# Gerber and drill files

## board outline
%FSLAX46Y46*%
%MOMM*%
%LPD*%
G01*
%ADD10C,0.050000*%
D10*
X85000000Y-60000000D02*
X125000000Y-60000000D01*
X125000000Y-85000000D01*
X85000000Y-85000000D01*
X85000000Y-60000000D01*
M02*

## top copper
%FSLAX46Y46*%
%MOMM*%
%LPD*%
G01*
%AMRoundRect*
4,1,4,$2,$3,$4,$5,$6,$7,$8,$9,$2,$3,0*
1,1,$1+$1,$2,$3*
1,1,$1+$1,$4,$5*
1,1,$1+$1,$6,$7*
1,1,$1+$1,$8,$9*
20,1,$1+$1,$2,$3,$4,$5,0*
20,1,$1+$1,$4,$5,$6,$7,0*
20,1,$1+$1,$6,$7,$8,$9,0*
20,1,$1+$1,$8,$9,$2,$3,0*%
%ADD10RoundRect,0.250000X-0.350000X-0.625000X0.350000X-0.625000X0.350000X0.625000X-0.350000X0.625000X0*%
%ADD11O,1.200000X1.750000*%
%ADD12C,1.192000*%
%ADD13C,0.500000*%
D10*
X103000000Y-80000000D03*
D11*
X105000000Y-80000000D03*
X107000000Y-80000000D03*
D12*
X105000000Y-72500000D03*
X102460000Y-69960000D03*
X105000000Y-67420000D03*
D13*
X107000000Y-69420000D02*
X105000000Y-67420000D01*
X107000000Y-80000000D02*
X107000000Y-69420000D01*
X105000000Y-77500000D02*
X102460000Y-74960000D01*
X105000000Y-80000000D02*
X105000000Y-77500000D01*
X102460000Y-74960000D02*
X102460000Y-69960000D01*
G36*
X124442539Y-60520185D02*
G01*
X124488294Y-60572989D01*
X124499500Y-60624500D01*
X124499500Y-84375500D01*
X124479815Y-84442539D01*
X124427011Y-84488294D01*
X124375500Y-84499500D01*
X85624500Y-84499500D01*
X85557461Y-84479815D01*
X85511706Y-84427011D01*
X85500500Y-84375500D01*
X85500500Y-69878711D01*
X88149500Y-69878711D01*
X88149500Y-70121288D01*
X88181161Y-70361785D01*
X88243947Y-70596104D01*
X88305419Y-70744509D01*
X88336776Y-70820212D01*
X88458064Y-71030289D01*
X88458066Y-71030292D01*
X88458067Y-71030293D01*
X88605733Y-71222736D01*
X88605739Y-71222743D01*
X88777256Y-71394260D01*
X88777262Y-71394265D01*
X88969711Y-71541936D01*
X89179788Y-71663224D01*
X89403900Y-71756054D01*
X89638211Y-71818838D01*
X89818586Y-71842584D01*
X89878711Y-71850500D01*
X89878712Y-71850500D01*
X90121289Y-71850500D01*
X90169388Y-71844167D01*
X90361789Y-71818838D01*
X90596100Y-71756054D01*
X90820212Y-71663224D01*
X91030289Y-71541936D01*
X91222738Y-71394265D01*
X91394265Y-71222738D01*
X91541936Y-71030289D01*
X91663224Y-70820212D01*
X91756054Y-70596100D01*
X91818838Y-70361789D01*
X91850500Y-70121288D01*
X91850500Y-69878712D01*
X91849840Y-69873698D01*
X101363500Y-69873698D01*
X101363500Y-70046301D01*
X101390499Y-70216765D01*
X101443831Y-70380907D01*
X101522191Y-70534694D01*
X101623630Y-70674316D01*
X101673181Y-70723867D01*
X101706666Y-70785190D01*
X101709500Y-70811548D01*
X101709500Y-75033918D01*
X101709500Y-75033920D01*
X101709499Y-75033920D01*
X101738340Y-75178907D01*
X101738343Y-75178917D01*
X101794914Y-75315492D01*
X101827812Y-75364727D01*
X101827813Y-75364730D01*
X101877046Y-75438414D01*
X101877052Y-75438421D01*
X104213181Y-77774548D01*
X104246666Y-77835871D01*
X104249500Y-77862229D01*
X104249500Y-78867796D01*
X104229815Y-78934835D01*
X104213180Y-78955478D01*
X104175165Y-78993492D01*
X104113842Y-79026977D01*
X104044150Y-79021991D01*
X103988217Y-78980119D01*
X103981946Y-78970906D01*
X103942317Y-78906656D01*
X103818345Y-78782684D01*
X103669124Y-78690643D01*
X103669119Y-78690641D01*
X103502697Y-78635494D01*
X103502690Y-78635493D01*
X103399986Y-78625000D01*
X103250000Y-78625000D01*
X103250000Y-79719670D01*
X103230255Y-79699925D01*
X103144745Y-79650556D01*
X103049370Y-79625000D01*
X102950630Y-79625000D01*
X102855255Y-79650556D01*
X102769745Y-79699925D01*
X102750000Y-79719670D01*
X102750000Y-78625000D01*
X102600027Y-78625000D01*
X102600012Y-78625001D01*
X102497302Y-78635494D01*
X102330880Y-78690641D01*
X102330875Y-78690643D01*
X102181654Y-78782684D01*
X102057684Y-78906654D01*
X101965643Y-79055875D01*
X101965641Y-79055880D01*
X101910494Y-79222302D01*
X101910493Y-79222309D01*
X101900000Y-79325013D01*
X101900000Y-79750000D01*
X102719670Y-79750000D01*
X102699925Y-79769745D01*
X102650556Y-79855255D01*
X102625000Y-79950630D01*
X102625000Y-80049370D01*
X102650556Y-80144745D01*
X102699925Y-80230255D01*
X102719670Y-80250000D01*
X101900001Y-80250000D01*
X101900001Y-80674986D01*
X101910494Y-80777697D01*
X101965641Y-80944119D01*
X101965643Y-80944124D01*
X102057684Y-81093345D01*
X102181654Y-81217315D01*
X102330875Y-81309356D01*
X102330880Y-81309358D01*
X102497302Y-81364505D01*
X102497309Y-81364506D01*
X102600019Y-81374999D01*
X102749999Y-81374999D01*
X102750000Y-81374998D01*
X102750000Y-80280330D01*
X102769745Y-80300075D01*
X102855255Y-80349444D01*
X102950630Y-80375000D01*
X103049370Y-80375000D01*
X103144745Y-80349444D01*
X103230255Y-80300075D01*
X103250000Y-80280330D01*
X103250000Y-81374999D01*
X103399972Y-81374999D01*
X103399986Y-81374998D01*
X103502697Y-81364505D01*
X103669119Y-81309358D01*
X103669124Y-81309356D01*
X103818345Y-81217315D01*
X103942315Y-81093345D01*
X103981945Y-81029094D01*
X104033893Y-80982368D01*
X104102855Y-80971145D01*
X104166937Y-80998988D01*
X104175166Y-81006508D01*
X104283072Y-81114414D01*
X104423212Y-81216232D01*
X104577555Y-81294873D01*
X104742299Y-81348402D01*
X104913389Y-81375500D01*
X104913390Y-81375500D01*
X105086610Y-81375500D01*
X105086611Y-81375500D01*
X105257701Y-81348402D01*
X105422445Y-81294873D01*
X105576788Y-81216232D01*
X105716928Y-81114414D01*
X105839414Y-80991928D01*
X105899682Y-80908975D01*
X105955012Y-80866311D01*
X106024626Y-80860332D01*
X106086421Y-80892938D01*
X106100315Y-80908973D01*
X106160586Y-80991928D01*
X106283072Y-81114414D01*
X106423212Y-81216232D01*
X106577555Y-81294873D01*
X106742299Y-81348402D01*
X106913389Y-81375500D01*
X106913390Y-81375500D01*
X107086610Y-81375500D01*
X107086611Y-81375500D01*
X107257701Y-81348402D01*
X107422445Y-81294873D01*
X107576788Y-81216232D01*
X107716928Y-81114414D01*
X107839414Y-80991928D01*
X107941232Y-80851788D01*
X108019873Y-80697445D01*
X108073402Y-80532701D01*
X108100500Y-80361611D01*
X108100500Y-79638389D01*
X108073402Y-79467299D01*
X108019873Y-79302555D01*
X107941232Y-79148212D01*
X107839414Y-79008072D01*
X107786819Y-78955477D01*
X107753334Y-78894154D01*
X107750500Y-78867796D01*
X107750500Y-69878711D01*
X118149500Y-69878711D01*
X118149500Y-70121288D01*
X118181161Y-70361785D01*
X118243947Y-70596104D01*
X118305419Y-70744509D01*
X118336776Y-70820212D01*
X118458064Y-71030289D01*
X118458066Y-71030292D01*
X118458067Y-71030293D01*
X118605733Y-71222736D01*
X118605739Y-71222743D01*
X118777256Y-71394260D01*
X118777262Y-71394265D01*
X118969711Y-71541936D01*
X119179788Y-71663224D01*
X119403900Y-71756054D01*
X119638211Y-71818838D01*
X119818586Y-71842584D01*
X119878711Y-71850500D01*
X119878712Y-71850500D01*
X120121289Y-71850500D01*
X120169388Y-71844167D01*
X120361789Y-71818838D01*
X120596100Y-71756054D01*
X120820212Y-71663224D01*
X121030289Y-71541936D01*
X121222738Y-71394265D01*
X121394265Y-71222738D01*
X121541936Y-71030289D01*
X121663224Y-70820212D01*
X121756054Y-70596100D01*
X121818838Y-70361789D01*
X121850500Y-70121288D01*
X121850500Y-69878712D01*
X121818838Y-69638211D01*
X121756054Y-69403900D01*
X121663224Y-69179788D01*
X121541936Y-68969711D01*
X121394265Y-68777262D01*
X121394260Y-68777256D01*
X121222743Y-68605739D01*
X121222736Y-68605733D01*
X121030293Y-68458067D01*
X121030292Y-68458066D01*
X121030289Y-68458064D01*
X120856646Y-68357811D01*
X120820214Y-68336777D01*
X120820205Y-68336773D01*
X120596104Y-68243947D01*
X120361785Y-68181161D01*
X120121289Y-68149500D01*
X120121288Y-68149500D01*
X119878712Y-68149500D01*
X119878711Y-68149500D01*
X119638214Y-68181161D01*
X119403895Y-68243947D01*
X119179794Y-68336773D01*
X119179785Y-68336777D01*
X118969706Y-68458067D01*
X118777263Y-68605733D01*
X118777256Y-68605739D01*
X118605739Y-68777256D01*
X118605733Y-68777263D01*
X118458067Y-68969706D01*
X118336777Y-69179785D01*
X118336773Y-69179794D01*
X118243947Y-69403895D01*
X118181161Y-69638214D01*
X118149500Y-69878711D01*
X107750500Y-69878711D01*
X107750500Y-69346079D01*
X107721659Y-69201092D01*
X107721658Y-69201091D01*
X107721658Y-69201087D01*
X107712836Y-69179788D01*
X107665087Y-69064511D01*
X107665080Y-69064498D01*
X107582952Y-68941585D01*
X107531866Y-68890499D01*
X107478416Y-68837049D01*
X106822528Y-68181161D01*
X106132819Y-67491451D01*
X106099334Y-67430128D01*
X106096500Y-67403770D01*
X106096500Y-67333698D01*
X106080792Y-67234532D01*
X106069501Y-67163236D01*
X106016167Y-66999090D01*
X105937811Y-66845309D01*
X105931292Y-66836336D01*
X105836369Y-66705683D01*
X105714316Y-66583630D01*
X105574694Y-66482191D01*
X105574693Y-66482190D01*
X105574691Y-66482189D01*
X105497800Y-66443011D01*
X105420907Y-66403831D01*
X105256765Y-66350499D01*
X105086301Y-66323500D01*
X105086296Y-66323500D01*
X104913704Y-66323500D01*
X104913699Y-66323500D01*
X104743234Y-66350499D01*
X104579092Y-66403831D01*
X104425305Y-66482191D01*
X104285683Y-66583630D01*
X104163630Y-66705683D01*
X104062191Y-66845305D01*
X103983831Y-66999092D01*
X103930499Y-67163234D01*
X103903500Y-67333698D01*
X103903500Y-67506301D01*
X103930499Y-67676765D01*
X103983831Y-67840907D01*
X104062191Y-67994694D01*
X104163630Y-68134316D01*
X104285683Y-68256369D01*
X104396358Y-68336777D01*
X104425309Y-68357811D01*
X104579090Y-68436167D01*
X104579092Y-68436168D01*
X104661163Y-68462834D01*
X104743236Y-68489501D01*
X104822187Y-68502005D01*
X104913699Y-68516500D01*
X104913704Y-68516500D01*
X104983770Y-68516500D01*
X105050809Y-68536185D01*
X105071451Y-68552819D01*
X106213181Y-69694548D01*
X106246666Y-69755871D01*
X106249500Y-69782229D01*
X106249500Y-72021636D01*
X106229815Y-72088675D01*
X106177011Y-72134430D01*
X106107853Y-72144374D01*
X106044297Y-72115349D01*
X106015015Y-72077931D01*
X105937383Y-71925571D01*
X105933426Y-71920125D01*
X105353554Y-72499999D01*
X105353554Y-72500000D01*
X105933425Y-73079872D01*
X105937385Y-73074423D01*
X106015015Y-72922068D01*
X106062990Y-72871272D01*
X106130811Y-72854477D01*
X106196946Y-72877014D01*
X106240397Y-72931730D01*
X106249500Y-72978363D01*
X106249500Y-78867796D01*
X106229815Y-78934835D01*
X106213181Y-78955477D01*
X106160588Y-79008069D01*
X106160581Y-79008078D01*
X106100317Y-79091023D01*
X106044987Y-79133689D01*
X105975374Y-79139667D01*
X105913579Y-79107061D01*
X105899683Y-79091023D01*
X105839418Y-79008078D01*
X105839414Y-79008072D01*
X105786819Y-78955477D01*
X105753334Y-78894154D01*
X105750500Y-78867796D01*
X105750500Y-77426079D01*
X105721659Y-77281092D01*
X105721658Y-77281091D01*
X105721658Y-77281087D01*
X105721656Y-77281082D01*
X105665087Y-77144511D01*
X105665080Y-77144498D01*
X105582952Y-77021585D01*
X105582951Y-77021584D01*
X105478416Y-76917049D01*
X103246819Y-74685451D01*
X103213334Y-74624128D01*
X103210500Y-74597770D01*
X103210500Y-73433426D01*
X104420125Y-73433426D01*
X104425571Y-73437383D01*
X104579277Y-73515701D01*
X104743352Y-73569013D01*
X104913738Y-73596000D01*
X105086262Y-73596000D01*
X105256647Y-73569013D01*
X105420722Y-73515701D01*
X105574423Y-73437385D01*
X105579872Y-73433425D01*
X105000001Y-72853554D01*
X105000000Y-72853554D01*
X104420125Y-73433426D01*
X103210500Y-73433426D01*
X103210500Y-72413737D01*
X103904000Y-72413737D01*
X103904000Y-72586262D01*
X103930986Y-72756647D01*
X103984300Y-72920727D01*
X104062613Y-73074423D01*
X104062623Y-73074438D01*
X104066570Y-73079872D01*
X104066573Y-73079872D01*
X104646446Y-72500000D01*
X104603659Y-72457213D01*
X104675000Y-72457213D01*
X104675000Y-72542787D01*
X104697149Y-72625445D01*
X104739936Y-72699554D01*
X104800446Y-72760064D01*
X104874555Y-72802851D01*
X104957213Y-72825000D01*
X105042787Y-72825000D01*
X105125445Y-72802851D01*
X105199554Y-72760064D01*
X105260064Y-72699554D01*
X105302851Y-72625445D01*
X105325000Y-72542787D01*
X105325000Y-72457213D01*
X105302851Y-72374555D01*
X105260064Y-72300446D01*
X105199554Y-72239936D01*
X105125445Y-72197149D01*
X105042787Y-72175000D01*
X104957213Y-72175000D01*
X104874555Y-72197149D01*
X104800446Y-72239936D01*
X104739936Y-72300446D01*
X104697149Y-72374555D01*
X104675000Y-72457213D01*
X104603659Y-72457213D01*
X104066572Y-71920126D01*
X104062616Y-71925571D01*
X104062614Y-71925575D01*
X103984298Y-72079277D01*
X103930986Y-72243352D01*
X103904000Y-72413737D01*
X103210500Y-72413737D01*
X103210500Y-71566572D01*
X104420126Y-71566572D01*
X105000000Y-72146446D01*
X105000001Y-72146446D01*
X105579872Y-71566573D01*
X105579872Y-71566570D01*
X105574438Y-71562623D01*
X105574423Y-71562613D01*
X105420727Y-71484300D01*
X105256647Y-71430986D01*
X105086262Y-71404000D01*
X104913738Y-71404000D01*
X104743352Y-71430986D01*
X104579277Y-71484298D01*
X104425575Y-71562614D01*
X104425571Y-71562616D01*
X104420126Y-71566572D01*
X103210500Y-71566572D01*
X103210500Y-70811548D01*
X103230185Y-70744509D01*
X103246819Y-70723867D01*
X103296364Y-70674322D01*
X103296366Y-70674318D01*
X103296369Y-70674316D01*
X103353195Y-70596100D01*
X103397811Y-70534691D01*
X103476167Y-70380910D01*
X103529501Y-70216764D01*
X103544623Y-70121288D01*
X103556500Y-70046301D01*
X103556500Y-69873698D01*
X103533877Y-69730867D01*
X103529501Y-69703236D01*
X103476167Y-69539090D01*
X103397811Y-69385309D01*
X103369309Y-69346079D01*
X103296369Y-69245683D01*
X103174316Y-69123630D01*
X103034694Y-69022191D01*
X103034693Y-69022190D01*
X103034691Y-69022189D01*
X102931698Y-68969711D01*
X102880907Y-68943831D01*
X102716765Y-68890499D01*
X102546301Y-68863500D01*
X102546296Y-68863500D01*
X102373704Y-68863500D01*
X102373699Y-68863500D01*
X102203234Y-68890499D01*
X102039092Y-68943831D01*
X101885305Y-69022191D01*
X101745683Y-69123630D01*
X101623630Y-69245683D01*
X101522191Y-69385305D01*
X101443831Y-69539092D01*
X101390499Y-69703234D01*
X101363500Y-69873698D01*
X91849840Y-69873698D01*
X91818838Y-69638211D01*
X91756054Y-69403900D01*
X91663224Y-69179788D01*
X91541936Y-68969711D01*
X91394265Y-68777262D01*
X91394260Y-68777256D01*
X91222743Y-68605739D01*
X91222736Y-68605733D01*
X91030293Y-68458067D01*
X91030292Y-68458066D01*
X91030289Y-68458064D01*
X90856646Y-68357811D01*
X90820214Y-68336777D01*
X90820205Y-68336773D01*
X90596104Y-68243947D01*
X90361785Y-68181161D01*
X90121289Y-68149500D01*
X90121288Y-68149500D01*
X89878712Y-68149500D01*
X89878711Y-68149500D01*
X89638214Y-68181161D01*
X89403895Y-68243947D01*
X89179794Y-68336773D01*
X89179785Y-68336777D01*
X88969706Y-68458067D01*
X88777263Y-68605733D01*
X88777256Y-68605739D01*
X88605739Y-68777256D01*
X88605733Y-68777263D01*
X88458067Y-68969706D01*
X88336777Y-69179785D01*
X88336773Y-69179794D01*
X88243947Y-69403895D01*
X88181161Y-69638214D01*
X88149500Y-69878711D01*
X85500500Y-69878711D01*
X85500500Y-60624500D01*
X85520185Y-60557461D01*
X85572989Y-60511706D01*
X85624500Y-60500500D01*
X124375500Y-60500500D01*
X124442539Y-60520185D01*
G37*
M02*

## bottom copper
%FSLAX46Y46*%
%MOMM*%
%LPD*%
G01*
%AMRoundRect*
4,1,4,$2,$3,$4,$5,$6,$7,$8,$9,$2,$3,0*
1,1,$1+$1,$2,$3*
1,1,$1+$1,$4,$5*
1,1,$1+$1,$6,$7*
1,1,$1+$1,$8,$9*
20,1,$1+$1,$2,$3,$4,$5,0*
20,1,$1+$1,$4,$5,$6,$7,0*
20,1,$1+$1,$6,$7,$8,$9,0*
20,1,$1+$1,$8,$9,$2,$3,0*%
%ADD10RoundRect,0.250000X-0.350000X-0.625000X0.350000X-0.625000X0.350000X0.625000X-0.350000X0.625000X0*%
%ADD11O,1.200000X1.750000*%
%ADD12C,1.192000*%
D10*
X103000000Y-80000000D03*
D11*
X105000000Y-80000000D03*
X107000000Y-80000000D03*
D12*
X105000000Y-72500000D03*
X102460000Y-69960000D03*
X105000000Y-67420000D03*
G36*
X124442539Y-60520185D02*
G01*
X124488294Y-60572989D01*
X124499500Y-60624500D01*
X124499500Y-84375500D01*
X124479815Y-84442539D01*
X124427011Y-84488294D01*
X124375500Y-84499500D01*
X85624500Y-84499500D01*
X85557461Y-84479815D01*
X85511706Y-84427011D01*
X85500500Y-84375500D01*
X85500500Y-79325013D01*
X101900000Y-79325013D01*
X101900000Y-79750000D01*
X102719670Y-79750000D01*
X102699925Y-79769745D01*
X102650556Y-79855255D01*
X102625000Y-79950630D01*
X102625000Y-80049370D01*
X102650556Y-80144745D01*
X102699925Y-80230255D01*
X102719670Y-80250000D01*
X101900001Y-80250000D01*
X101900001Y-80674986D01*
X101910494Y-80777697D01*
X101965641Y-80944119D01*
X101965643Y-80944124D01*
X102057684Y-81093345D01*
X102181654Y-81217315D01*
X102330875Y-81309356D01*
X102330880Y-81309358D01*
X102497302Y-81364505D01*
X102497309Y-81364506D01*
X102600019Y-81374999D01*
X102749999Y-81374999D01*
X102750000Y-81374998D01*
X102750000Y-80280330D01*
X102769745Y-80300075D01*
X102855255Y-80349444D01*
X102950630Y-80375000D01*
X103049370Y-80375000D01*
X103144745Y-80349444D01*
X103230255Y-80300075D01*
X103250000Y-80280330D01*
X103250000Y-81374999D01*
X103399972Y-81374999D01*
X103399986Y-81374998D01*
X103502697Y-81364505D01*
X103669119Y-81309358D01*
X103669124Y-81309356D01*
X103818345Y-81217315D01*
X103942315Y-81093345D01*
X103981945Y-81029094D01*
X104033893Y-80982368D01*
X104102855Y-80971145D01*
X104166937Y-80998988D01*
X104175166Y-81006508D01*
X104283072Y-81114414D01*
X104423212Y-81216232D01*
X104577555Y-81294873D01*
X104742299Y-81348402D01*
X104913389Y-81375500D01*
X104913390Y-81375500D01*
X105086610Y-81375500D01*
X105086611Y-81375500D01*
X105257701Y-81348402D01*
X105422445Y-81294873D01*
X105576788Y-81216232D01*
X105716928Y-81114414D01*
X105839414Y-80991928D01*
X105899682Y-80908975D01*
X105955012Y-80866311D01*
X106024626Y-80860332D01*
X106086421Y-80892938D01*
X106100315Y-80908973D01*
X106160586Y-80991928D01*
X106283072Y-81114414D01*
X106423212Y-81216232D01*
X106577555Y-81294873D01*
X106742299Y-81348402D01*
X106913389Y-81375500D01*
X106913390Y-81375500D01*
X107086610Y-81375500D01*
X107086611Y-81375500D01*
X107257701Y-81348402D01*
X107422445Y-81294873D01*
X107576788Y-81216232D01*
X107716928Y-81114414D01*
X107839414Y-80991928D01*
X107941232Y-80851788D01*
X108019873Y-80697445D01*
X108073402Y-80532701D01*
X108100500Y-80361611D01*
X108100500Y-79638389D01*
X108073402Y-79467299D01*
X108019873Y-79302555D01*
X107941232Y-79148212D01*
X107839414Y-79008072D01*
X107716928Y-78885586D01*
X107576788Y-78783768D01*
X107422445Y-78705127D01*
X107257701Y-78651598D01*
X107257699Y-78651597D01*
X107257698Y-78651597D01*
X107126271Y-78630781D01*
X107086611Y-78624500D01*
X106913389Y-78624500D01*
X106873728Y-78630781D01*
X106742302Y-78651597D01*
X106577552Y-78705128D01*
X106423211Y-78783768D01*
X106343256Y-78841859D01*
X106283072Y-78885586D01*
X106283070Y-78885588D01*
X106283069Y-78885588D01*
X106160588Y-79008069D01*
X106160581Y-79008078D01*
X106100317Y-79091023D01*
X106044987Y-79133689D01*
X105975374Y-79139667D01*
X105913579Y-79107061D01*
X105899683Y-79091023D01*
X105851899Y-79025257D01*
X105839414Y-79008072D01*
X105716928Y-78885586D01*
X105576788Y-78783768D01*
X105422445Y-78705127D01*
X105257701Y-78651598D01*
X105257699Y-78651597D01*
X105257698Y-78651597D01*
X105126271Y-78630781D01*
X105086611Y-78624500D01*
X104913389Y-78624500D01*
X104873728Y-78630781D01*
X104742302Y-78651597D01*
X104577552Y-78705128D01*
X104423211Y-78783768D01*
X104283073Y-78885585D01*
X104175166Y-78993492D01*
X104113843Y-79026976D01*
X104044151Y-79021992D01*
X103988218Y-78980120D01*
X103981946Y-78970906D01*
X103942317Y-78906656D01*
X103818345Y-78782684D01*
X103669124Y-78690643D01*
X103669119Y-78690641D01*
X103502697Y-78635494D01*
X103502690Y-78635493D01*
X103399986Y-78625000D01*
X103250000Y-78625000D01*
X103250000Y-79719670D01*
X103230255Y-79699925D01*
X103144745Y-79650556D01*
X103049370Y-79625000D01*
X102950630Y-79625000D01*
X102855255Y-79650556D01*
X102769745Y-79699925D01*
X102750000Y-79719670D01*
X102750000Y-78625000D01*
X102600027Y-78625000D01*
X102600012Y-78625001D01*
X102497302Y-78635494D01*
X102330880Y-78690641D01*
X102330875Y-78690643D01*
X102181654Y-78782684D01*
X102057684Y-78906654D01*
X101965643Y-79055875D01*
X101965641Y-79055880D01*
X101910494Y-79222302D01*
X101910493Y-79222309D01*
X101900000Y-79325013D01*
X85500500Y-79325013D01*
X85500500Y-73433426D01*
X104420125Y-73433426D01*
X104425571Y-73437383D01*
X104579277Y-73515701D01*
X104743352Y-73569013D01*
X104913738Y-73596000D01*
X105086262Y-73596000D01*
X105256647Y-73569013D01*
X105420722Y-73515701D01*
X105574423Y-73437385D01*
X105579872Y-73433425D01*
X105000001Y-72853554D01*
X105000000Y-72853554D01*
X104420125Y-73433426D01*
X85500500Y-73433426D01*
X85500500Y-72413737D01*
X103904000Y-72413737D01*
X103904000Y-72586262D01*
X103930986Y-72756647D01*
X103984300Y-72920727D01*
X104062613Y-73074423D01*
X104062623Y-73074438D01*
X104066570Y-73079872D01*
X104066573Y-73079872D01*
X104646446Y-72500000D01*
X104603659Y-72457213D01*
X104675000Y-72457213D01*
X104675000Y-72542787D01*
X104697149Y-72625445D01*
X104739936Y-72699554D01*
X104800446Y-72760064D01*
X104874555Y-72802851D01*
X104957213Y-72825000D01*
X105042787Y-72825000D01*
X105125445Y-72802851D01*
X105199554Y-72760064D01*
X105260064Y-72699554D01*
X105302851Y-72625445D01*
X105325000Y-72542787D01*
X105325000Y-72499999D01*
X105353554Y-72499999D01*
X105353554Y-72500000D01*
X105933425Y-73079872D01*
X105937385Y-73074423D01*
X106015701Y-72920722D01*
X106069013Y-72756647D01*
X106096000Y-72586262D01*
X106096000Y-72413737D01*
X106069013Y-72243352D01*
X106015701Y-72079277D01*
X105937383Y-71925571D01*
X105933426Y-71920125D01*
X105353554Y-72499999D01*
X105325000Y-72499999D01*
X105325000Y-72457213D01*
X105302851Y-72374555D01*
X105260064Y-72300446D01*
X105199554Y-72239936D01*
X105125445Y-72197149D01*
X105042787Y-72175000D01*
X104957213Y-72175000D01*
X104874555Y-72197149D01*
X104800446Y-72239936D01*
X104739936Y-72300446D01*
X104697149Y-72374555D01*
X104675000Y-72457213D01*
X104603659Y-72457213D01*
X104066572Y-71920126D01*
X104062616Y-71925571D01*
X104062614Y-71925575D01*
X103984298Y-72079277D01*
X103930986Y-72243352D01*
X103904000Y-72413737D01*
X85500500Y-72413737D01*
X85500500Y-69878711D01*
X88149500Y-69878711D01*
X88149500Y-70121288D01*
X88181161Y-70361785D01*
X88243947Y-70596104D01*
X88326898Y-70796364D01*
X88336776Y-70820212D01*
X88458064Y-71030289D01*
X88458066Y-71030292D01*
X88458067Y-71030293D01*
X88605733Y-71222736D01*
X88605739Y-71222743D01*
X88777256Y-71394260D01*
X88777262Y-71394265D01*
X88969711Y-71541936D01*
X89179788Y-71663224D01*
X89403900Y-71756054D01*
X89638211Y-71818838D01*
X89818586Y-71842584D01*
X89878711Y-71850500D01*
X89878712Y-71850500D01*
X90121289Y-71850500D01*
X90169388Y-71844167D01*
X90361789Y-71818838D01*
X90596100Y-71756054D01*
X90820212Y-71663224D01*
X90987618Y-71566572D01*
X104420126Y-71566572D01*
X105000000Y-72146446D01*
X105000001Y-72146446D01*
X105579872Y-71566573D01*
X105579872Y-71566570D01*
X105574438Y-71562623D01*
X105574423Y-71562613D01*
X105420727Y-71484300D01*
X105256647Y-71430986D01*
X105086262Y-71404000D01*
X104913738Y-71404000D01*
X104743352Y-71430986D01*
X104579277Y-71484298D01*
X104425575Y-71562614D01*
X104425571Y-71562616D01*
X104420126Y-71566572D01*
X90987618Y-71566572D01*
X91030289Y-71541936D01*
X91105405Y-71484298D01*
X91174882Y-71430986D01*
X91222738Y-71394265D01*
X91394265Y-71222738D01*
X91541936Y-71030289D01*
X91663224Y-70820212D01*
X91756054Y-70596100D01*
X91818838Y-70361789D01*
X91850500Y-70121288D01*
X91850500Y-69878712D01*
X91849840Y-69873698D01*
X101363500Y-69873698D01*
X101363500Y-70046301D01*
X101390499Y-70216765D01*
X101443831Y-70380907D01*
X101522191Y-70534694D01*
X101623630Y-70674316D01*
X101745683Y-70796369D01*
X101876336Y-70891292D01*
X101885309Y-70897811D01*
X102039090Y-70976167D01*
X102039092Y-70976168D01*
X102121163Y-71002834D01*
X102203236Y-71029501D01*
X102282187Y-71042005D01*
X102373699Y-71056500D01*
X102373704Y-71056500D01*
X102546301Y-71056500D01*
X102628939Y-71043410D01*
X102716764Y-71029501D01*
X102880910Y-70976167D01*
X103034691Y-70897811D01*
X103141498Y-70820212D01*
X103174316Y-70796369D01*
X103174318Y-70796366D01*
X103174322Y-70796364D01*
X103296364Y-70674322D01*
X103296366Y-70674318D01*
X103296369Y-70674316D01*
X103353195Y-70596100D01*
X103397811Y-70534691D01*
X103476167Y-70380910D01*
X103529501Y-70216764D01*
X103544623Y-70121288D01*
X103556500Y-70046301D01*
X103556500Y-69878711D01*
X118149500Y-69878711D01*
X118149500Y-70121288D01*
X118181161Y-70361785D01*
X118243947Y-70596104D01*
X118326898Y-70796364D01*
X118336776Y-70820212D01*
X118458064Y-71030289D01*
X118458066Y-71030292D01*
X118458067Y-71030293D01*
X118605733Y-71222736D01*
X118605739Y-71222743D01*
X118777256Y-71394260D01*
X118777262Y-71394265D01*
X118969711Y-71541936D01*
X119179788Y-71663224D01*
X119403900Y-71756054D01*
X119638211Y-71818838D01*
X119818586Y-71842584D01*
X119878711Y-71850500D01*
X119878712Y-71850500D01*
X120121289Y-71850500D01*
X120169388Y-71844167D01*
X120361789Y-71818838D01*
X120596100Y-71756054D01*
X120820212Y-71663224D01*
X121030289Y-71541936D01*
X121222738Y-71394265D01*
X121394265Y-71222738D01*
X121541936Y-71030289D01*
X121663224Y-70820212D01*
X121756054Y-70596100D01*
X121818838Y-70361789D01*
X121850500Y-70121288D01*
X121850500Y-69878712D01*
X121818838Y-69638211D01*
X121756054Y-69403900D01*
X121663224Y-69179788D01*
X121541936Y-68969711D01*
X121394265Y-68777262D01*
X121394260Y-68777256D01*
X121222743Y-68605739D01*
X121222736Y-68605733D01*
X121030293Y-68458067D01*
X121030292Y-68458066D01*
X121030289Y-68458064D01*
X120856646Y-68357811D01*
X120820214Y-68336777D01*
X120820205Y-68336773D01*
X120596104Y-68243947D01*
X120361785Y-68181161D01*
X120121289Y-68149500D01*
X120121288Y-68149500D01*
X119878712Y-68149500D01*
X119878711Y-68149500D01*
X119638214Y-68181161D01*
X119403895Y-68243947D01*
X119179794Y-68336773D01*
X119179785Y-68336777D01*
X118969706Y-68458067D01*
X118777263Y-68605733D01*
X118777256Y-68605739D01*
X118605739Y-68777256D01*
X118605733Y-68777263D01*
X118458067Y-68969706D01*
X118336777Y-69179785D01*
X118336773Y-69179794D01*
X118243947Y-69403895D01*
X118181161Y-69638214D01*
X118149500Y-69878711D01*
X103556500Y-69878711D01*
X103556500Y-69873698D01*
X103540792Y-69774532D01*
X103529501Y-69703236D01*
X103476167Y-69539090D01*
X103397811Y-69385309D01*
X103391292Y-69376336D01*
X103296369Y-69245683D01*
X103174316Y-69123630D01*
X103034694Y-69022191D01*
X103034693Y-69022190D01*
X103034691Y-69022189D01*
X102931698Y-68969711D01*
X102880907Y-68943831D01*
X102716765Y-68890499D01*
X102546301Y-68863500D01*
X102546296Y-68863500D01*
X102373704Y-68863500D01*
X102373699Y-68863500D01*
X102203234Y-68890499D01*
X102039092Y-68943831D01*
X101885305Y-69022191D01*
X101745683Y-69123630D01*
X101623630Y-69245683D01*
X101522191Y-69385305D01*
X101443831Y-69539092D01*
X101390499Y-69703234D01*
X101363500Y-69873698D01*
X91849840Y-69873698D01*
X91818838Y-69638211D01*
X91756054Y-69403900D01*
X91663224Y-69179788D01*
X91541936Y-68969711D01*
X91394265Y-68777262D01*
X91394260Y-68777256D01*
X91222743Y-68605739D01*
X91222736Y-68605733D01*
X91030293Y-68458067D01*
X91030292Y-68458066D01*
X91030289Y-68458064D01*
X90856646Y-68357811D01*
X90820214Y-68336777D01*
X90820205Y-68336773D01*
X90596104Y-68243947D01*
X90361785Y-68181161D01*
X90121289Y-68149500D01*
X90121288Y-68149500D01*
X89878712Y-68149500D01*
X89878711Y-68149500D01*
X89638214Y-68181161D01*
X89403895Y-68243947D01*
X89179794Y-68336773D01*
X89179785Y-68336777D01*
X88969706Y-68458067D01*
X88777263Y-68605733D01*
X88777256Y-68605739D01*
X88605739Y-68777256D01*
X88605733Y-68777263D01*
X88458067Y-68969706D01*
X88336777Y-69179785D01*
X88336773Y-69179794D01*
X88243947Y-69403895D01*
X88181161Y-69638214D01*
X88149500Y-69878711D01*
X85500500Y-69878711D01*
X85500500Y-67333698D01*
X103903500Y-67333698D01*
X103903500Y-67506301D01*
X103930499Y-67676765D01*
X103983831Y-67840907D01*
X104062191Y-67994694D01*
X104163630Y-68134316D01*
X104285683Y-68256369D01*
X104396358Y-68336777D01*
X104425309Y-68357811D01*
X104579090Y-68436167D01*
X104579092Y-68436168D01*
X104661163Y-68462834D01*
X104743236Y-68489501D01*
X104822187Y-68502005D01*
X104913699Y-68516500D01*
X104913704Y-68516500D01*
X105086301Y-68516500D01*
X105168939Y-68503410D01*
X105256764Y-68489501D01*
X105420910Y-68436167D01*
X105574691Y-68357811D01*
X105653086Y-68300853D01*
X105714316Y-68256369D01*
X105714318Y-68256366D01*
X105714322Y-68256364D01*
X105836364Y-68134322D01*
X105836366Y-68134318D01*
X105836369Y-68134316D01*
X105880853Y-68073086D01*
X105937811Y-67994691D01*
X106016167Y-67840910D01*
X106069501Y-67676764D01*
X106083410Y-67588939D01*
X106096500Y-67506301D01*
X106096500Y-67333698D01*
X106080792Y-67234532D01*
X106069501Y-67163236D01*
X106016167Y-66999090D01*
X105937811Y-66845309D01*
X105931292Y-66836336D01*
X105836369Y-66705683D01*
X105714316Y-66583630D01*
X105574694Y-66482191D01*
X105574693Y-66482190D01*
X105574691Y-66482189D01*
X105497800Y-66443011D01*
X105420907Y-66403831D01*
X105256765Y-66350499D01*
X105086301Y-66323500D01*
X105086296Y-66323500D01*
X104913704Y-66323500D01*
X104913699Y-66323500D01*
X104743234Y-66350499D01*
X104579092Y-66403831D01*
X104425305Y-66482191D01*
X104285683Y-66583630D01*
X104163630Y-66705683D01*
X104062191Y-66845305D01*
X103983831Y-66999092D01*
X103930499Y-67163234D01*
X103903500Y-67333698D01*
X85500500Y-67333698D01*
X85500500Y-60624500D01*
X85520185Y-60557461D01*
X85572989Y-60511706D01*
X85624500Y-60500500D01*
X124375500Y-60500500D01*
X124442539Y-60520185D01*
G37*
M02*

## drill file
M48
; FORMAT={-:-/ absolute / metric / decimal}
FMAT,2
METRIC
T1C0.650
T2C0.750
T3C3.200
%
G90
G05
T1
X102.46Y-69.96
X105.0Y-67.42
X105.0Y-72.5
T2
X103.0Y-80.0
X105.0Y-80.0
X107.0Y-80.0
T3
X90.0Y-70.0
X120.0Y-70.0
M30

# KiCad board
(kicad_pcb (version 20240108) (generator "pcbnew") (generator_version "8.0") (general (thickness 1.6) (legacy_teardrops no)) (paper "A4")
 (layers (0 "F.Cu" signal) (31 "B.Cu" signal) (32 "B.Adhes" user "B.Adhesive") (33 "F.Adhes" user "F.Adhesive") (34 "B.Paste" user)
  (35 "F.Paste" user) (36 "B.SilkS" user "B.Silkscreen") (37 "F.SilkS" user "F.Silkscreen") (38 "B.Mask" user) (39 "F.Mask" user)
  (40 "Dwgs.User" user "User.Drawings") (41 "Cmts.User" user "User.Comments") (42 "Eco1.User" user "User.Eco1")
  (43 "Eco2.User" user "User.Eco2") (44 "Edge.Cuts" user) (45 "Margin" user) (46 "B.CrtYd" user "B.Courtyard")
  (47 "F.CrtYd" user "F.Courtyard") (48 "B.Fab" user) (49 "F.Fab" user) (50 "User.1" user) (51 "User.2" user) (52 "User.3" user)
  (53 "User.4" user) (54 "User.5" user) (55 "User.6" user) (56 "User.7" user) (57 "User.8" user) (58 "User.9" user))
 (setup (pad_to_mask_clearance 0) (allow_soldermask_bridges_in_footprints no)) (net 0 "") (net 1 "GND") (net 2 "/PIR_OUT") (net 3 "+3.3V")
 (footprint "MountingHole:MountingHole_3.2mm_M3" (layer "F.Cu") (at 120 70)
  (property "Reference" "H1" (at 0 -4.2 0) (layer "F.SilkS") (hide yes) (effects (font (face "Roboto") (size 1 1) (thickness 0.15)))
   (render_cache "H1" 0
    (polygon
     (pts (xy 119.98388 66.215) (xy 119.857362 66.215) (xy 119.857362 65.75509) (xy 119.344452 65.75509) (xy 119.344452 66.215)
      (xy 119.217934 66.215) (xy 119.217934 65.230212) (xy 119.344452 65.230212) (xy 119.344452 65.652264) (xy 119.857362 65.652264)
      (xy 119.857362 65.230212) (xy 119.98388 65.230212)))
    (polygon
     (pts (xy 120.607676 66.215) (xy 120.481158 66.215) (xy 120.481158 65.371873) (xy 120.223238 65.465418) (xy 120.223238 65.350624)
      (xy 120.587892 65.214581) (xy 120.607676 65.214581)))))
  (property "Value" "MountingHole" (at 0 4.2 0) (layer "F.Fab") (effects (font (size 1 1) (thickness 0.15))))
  (pad "" np_thru_hole circle (at 0 0) (size 3.2 3.2) (drill 3.2) (layers "*.Cu" "*.Mask")))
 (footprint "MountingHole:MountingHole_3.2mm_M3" (layer "F.Cu") (at 90 70)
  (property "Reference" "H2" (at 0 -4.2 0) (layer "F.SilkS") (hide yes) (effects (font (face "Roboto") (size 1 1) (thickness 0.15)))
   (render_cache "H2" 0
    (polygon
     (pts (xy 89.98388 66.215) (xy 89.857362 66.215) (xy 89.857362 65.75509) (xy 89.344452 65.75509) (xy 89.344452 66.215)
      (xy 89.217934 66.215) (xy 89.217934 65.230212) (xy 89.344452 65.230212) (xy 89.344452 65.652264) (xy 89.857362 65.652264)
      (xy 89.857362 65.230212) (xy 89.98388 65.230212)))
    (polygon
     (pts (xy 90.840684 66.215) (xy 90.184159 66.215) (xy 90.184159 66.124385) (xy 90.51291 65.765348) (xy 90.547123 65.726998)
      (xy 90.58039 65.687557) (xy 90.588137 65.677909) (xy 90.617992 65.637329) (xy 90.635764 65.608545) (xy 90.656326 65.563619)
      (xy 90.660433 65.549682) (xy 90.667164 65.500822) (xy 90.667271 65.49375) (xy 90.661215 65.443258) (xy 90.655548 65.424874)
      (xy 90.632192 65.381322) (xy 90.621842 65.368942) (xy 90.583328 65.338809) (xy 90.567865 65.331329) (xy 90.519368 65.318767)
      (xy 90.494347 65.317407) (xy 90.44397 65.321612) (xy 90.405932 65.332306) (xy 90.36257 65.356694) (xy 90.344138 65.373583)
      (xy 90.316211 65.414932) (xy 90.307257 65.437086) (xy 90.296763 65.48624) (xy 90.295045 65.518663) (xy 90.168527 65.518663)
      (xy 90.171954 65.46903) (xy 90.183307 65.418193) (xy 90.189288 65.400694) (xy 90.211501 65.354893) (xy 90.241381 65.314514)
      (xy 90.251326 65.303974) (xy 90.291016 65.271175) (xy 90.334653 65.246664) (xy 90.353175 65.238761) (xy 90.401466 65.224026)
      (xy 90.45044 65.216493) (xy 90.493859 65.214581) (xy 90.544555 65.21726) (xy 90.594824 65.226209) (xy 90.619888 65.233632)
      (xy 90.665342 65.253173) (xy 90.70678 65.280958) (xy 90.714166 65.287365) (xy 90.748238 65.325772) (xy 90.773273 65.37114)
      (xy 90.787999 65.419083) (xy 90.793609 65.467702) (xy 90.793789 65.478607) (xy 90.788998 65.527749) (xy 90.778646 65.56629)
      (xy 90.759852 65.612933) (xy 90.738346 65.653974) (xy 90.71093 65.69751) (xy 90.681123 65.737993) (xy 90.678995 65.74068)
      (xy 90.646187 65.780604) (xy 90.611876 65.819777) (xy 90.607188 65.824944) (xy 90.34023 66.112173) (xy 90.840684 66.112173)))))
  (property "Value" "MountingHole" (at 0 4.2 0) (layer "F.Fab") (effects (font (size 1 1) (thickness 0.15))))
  (pad "" np_thru_hole circle (at 0 0) (size 3.2 3.2) (drill 3.2) (layers "*.Cu" "*.Mask")))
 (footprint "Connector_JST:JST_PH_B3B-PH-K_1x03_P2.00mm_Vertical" (layer "F.Cu") (at 103 80)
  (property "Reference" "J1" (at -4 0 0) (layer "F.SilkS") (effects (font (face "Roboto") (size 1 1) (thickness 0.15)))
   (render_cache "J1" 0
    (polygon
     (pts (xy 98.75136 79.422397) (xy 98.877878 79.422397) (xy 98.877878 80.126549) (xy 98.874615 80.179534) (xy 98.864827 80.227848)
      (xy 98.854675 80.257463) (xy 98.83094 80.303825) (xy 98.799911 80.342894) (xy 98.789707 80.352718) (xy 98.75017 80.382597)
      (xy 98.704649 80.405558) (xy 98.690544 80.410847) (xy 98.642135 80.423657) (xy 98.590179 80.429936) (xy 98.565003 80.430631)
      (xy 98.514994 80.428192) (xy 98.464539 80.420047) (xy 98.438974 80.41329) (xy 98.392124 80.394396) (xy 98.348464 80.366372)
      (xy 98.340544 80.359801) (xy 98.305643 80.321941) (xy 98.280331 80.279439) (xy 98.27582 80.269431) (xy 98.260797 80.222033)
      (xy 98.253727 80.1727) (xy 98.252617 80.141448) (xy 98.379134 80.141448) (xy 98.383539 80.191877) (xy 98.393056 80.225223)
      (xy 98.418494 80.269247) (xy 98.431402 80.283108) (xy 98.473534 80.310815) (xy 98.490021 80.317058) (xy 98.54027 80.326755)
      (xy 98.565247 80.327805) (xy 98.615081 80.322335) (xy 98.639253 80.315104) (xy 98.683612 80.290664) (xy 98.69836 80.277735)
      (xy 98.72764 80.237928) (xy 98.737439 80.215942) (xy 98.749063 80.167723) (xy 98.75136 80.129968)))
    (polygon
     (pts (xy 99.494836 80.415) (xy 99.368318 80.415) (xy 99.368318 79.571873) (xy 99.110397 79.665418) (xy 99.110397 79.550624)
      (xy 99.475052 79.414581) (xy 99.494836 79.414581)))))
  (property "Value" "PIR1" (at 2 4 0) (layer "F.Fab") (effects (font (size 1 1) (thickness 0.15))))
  (pad "1" thru_hole roundrect (at 0 0) (size 1.2 1.75) (drill 0.75) (layers "*.Cu" "*.Mask") (remove_unused_layers no)
   (roundrect_rratio 0.208333) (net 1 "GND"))
  (pad "2" thru_hole oval (at 2 0) (size 1.2 1.75) (drill 0.75) (layers "*.Cu" "*.Mask") (remove_unused_layers no) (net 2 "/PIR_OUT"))
  (pad "3" thru_hole oval (at 4 0) (size 1.2 1.75) (drill 0.75) (layers "*.Cu" "*.Mask") (remove_unused_layers no) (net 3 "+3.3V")))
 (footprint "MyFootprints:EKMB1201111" (layer "B.Cu") (at 105 72.5 180)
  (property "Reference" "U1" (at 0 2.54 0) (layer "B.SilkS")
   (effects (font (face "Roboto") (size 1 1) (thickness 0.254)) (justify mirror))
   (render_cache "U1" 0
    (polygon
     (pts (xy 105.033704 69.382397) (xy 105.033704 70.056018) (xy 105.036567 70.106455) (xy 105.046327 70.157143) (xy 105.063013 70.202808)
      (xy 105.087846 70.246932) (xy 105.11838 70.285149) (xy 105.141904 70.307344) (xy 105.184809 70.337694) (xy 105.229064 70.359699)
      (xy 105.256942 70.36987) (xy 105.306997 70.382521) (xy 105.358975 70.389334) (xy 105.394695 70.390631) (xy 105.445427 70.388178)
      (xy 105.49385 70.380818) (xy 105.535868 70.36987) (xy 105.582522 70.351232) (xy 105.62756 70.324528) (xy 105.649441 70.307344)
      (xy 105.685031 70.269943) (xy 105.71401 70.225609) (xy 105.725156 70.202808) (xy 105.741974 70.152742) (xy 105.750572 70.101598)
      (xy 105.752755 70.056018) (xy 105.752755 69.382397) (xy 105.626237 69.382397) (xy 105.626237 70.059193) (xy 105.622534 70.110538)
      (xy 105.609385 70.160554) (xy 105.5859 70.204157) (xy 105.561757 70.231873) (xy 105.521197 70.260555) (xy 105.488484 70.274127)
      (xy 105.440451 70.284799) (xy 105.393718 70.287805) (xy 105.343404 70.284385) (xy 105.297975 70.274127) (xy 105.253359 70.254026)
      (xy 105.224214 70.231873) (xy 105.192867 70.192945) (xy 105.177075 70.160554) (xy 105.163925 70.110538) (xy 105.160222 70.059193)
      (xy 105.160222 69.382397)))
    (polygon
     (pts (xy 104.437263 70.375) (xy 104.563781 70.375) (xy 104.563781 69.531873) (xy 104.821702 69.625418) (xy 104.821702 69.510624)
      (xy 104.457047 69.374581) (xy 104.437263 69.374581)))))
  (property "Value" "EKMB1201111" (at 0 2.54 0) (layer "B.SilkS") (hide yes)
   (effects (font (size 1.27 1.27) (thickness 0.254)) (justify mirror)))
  (pad "1" thru_hole circle (at 0 0 180) (size 1.192 1.192) (drill 0.65) (layers "*.Cu" "*.Mask") (remove_unused_layers no) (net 1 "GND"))
  (pad "2" thru_hole circle (at 2.54 2.54 180) (size 1.192 1.192) (drill 0.65) (layers "*.Cu" "*.Mask") (remove_unused_layers no)
   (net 2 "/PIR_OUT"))
  (pad "3" thru_hole circle (at 0 5.08 180) (size 1.192 1.192) (drill 0.65) (layers "*.Cu" "*.Mask") (remove_unused_layers no)
   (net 3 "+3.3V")))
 (gr_rect (start 85 60) (end 125 85) (stroke (width 0.05) (type default)) (fill none) (layer "Edge.Cuts"))
 (segment (start 107 69.42) (end 105 67.42) (width 0.5) (layer "F.Cu") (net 3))
 (segment (start 107 80) (end 107 69.42) (width 0.5) (layer "F.Cu") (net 3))
 (segment (start 105 77.5) (end 102.46 74.96) (width 0.5) (layer "F.Cu") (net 2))
 (segment (start 105 80) (end 105 77.5) (width 0.5) (layer "F.Cu") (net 2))
 (segment (start 102.46 74.96) (end 102.46 69.96) (width 0.5) (layer "F.Cu") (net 2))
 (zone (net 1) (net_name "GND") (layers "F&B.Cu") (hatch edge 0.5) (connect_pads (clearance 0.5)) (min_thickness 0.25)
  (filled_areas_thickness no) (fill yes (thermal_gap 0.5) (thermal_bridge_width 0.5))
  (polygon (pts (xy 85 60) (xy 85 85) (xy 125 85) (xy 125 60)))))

